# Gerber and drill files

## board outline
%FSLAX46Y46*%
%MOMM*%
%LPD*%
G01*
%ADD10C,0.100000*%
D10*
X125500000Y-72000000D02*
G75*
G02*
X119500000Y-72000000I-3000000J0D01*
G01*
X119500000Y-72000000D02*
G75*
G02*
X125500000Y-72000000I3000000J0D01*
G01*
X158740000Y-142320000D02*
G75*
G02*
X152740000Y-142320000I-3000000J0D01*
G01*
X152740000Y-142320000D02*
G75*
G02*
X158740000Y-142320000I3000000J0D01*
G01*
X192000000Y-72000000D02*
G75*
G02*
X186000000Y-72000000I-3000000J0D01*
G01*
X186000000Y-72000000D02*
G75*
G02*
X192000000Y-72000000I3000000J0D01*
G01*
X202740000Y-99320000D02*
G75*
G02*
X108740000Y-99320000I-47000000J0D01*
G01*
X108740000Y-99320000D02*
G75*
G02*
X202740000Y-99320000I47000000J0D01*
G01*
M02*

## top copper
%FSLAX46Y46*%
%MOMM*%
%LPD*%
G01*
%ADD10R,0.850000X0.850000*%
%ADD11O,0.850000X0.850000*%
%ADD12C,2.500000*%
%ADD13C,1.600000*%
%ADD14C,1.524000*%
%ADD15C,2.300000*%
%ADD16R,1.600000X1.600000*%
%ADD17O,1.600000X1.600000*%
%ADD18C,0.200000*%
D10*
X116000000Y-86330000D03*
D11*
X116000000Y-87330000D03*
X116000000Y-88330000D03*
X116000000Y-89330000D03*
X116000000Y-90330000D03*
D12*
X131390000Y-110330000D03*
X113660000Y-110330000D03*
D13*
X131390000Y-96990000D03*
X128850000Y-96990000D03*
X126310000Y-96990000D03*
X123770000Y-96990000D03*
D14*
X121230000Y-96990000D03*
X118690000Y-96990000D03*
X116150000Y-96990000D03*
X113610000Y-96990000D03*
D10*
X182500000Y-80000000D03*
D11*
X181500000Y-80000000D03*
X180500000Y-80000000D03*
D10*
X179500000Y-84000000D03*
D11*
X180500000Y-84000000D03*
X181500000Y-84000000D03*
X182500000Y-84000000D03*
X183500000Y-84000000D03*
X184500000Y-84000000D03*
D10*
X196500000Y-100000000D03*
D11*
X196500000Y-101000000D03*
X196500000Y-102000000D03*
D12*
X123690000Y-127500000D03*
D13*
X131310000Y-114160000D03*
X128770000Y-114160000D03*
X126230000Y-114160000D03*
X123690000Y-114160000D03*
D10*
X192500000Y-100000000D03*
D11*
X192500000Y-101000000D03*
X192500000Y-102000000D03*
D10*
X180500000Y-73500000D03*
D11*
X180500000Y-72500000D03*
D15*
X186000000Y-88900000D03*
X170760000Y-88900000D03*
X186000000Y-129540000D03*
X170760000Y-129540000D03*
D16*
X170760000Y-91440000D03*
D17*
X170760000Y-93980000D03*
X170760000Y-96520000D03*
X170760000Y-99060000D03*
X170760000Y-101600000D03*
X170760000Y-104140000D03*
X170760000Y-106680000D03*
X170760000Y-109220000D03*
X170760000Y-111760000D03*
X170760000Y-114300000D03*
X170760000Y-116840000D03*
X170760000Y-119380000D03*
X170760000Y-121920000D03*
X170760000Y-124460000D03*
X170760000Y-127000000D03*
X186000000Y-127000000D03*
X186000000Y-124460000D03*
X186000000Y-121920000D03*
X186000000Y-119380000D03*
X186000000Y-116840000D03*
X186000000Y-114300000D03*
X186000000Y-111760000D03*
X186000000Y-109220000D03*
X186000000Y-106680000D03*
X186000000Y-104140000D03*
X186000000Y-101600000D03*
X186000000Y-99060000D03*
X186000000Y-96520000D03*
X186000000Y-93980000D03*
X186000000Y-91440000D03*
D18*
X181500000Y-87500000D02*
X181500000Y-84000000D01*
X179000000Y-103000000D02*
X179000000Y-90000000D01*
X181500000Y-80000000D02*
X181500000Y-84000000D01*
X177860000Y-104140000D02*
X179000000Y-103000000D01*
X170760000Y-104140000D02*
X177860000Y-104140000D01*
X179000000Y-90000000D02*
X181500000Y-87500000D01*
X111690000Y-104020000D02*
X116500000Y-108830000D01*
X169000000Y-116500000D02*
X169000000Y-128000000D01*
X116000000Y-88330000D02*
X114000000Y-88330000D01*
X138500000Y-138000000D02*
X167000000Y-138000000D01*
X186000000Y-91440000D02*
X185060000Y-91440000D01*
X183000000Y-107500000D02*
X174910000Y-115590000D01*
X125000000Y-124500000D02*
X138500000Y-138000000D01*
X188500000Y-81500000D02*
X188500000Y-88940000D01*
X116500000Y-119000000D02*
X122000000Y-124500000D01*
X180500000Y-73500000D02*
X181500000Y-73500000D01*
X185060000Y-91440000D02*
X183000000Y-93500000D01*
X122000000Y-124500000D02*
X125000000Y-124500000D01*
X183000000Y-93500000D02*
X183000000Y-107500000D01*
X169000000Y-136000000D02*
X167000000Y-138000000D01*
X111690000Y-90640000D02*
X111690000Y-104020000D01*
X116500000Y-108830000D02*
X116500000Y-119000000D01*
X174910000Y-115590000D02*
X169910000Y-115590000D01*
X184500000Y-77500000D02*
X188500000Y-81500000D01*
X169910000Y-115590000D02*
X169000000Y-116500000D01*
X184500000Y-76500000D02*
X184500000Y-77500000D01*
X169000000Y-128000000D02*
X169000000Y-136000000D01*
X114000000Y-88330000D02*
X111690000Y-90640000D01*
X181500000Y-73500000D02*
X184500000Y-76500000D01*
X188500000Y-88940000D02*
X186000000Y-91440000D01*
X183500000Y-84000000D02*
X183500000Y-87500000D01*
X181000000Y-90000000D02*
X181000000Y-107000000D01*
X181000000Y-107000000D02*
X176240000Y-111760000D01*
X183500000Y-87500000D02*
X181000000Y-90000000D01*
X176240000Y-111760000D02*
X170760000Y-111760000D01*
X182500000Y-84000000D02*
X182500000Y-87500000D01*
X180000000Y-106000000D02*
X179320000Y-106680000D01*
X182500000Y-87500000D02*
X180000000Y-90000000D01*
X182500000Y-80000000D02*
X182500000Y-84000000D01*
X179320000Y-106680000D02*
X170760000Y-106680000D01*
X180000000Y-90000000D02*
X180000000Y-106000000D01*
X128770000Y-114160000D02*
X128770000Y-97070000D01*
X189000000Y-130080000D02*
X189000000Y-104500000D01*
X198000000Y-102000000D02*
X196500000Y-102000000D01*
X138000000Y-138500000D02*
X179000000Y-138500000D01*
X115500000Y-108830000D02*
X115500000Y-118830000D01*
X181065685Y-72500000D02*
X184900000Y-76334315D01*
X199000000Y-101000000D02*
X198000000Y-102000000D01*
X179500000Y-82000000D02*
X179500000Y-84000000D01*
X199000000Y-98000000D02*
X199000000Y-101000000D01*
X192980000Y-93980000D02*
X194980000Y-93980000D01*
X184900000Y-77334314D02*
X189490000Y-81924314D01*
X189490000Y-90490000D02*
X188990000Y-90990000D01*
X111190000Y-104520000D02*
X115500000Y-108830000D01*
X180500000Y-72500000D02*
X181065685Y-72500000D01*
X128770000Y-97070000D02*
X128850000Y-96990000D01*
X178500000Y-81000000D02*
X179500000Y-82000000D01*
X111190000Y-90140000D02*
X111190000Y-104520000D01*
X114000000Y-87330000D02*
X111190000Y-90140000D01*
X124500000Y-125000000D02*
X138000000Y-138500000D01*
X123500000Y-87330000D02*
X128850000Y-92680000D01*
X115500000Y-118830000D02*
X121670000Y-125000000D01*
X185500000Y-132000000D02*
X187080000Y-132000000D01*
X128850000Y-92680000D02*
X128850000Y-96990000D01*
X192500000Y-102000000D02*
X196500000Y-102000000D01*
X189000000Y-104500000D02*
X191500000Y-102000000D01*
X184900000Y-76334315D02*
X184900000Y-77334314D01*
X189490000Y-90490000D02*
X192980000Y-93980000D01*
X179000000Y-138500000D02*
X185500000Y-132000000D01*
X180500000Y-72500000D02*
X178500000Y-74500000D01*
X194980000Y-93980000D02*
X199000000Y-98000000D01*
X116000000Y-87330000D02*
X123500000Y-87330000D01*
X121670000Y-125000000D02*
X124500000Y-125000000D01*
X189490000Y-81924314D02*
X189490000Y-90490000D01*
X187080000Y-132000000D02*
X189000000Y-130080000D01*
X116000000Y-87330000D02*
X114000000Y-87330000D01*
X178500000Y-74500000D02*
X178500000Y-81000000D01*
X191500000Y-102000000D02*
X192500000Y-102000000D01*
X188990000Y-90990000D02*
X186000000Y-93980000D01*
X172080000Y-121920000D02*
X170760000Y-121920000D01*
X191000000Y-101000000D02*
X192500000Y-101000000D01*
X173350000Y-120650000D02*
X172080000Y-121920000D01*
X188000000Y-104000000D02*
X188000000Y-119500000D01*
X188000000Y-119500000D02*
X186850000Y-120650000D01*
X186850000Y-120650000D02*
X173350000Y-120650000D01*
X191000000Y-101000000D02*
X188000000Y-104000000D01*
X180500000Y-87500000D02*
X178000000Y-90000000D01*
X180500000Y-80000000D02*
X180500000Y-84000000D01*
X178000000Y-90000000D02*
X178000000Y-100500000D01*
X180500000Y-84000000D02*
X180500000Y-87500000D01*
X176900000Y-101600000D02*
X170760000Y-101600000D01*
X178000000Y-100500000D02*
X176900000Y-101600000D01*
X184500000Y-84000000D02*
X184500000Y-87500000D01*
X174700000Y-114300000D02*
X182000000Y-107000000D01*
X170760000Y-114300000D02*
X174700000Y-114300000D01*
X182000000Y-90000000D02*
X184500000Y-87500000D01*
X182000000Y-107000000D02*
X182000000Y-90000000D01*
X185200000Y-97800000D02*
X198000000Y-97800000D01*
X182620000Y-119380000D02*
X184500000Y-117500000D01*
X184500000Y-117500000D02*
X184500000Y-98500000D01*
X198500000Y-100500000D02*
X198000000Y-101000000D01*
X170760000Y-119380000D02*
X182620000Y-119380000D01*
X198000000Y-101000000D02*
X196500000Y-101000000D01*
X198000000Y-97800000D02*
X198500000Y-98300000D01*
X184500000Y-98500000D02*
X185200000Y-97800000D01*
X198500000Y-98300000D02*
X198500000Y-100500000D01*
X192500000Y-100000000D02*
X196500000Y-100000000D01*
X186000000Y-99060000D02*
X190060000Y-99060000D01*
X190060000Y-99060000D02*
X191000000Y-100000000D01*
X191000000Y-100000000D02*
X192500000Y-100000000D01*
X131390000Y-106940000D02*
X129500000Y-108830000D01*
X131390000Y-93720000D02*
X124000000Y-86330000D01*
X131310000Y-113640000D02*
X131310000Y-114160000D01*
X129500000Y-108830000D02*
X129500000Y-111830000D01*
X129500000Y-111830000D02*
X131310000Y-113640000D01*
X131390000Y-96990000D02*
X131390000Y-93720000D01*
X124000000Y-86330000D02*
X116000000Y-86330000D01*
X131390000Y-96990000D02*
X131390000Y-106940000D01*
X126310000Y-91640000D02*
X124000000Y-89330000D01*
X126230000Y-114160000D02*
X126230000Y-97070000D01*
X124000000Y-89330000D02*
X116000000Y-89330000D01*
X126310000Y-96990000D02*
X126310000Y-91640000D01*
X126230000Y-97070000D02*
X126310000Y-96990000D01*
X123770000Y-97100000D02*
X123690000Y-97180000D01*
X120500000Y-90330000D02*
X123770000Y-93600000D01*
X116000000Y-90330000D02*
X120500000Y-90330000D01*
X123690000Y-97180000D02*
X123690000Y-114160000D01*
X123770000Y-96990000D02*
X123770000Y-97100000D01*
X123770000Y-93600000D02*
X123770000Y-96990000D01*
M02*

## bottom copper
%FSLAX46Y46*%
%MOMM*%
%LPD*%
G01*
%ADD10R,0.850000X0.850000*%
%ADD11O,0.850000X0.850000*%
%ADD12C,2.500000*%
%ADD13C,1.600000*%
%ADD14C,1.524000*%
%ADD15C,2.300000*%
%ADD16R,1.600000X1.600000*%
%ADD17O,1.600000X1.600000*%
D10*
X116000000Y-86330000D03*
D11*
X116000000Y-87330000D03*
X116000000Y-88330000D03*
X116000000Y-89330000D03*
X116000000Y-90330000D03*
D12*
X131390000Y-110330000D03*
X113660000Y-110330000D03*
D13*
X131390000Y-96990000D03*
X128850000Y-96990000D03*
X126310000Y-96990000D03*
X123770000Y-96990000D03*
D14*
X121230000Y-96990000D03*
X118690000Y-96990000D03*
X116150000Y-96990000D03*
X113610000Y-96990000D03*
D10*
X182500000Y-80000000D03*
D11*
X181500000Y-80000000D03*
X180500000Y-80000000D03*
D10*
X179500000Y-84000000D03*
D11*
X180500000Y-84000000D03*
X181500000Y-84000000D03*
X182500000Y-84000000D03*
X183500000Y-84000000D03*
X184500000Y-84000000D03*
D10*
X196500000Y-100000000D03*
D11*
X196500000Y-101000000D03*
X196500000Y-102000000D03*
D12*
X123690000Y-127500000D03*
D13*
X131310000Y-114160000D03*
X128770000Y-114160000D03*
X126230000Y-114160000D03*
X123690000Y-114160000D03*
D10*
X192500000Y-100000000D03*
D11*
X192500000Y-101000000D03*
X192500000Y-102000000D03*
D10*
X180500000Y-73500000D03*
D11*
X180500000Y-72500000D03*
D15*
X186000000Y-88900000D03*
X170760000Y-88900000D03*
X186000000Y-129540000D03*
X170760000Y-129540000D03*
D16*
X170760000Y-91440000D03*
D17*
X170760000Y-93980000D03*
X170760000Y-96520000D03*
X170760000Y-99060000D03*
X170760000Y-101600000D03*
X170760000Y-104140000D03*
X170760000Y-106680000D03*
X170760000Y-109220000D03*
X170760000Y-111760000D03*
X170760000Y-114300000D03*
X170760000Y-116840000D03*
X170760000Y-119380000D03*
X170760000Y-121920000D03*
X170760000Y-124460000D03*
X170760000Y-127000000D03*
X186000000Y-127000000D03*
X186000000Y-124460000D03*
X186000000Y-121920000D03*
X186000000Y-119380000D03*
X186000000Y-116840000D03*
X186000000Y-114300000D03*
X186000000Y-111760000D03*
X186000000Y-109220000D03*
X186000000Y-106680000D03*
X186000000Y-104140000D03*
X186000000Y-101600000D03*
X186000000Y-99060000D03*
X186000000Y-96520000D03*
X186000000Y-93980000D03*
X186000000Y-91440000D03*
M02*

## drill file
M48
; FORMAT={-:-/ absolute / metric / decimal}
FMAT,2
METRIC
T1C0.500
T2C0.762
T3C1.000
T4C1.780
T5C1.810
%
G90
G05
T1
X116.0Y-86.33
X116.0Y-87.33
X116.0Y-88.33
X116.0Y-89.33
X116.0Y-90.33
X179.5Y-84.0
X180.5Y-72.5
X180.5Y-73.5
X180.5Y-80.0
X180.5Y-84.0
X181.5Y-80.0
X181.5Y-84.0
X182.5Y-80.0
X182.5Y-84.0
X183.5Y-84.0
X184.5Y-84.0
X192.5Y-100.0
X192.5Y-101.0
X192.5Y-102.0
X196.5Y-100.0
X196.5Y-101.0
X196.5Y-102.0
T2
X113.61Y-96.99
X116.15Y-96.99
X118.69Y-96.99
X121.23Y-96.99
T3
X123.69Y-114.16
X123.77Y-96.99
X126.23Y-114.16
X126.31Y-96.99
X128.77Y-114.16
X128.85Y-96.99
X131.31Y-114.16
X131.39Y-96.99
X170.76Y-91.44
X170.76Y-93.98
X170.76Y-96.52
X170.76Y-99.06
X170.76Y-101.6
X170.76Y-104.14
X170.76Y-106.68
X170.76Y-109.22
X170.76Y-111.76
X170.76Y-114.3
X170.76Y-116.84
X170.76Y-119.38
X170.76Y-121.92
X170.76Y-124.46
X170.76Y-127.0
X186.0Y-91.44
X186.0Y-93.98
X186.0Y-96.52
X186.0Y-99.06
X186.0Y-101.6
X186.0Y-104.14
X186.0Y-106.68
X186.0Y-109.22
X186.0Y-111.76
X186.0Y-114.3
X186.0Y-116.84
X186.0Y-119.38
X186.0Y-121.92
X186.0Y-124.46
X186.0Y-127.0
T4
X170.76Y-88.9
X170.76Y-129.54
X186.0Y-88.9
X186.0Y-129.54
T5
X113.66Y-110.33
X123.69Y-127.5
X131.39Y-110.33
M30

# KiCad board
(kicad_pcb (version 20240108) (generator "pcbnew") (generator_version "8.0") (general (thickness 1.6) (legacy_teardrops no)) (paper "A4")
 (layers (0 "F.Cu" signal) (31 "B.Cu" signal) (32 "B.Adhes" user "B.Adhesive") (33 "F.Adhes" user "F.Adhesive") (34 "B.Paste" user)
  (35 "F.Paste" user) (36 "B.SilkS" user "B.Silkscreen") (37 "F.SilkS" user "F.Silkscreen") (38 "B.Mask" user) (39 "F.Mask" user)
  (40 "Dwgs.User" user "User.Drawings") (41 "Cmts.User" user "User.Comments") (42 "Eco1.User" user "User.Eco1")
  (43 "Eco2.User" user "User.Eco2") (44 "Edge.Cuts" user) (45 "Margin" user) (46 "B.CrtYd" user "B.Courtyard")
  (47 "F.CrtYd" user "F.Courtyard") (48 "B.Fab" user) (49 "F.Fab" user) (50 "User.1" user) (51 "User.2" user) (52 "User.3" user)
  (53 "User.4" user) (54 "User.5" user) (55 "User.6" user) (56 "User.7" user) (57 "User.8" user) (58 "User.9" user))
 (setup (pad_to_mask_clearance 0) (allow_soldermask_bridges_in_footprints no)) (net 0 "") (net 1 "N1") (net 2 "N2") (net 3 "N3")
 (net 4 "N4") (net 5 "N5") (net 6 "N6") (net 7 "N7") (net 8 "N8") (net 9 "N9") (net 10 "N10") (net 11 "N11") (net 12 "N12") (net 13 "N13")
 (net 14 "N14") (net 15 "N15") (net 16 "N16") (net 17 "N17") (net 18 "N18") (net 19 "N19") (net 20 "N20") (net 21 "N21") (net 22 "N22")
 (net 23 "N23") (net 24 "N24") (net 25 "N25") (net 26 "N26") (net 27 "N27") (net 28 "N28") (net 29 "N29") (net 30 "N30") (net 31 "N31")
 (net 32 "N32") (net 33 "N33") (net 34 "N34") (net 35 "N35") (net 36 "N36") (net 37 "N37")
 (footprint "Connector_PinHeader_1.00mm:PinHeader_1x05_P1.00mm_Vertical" (layer "F.Cu") (at 116 86.33)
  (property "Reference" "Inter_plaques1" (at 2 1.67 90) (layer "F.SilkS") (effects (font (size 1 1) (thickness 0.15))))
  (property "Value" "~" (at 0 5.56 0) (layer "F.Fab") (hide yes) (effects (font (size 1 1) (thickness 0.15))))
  (pad "1" thru_hole rect (at 0 0) (size 0.85 0.85) (drill 0.5) (layers "*.Cu" "*.Mask") (remove_unused_layers no) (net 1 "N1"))
  (pad "2" thru_hole oval (at 0 1) (size 0.85 0.85) (drill 0.5) (layers "*.Cu" "*.Mask") (remove_unused_layers no) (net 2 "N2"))
  (pad "3" thru_hole oval (at 0 2) (size 0.85 0.85) (drill 0.5) (layers "*.Cu" "*.Mask") (remove_unused_layers no) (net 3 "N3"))
  (pad "4" thru_hole oval (at 0 3) (size 0.85 0.85) (drill 0.5) (layers "*.Cu" "*.Mask") (remove_unused_layers no) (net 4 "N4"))
  (pad "5" thru_hole oval (at 0 4) (size 0.85 0.85) (drill 0.5) (layers "*.Cu" "*.Mask") (remove_unused_layers no) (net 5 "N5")))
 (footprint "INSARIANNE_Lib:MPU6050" (layer "F.Cu") (at 131.39 96.99 180)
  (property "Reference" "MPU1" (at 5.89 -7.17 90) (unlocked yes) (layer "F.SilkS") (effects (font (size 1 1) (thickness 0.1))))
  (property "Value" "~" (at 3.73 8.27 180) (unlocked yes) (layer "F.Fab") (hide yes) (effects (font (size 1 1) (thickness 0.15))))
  (pad "" np_thru_hole circle (at 0 -13.34 180) (size 2.5 2.5) (drill 1.81) (layers "F&B.Cu" "*.Mask"))
  (pad "" np_thru_hole circle (at 17.73 -13.34 180) (size 2.5 2.5) (drill 1.81) (layers "F&B.Cu" "*.Mask"))
  (pad "1" thru_hole circle (at 0 0 180) (size 1.6 1.6) (drill 1) (layers "*.Cu" "*.Mask") (remove_unused_layers no) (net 1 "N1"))
  (pad "2" thru_hole circle (at 2.54 0 180) (size 1.6 1.6) (drill 1) (layers "*.Cu" "*.Mask") (remove_unused_layers no) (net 2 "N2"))
  (pad "3" thru_hole circle (at 5.08 0 180) (size 1.6 1.6) (drill 1) (layers "*.Cu" "*.Mask") (remove_unused_layers no) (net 4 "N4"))
  (pad "4" thru_hole circle (at 7.62 0 180) (size 1.6 1.6) (drill 1) (layers "*.Cu" "*.Mask") (remove_unused_layers no) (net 5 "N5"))
  (pad "5" thru_hole circle (at 10.16 0 180) (size 1.524 1.524) (drill 0.762) (layers "*.Cu" "*.Mask") (remove_unused_layers no)
   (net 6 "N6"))
  (pad "6" thru_hole circle (at 12.7 0 180) (size 1.524 1.524) (drill 0.762) (layers "*.Cu" "*.Mask") (remove_unused_layers no) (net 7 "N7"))
  (pad "7" thru_hole circle (at 15.24 0 180) (size 1.524 1.524) (drill 0.762) (layers "*.Cu" "*.Mask") (remove_unused_layers no)
   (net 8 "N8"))
  (pad "8" thru_hole circle (at 17.78 0 180) (size 1.524 1.524) (drill 0.762) (layers "*.Cu" "*.Mask") (remove_unused_layers no)
   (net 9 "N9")))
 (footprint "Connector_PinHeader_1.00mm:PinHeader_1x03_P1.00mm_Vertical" (layer "F.Cu") (at 182.5 80 -90)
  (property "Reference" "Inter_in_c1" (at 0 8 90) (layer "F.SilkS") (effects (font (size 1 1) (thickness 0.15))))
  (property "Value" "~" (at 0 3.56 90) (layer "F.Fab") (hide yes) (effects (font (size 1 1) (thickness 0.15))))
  (pad "1" thru_hole rect (at 0 0 270) (size 0.85 0.85) (drill 0.5) (layers "*.Cu" "*.Mask") (remove_unused_layers no) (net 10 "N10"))
  (pad "2" thru_hole oval (at 0 1 270) (size 0.85 0.85) (drill 0.5) (layers "*.Cu" "*.Mask") (remove_unused_layers no) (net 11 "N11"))
  (pad "3" thru_hole oval (at 0 2 270) (size 0.85 0.85) (drill 0.5) (layers "*.Cu" "*.Mask") (remove_unused_layers no) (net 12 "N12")))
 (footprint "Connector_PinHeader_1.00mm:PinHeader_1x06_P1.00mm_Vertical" (layer "F.Cu") (at 179.5 84 90)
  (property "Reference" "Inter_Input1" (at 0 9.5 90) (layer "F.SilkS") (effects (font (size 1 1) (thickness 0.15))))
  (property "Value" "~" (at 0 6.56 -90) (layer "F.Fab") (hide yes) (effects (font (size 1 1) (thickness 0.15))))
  (pad "1" thru_hole rect (at 0 0 90) (size 0.85 0.85) (drill 0.5) (layers "*.Cu" "*.Mask") (remove_unused_layers no) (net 2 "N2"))
  (pad "2" thru_hole oval (at 0 1 90) (size 0.85 0.85) (drill 0.5) (layers "*.Cu" "*.Mask") (remove_unused_layers no) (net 12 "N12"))
  (pad "3" thru_hole oval (at 0 2 90) (size 0.85 0.85) (drill 0.5) (layers "*.Cu" "*.Mask") (remove_unused_layers no) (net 11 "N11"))
  (pad "4" thru_hole oval (at 0 3 90) (size 0.85 0.85) (drill 0.5) (layers "*.Cu" "*.Mask") (remove_unused_layers no) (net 10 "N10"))
  (pad "5" thru_hole oval (at 0 4 90) (size 0.85 0.85) (drill 0.5) (layers "*.Cu" "*.Mask") (remove_unused_layers no) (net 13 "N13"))
  (pad "6" thru_hole oval (at 0 5 90) (size 0.85 0.85) (drill 0.5) (layers "*.Cu" "*.Mask") (remove_unused_layers no) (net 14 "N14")))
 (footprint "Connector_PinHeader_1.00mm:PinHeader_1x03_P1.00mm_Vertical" (layer "F.Cu") (at 196.5 100)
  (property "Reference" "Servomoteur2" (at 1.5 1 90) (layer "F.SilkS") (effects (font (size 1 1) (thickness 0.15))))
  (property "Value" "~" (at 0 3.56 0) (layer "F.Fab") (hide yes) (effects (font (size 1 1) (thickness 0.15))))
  (pad "1" thru_hole rect (at 0 0) (size 0.85 0.85) (drill 0.5) (layers "*.Cu" "*.Mask") (remove_unused_layers no) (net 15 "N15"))
  (pad "2" thru_hole oval (at 0 1) (size 0.85 0.85) (drill 0.5) (layers "*.Cu" "*.Mask") (remove_unused_layers no) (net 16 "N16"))
  (pad "3" thru_hole oval (at 0 2) (size 0.85 0.85) (drill 0.5) (layers "*.Cu" "*.Mask") (remove_unused_layers no) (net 2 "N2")))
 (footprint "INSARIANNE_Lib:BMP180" (layer "F.Cu") (at 131.31 114.16 180)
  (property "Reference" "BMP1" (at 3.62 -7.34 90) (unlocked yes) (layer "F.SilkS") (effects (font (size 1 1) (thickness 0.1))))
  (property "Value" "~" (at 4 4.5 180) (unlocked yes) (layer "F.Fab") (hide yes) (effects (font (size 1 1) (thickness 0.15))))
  (pad "" np_thru_hole circle (at 7.62 -13.34 180) (size 2.5 2.5) (drill 1.81) (layers "F&B.Cu" "*.Mask"))
  (pad "1" thru_hole circle (at 0 0 180) (size 1.6 1.6) (drill 1) (layers "*.Cu" "*.Mask") (remove_unused_layers no) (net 1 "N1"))
  (pad "2" thru_hole circle (at 2.54 0 180) (size 1.6 1.6) (drill 1) (layers "*.Cu" "*.Mask") (remove_unused_layers no) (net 2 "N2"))
  (pad "3" thru_hole circle (at 5.08 0 180) (size 1.6 1.6) (drill 1) (layers "*.Cu" "*.Mask") (remove_unused_layers no) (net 4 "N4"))
  (pad "4" thru_hole circle (at 7.62 0 180) (size 1.6 1.6) (drill 1) (layers "*.Cu" "*.Mask") (remove_unused_layers no) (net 5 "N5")))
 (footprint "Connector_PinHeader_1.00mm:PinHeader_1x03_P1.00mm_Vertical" (layer "F.Cu") (at 192.5 100)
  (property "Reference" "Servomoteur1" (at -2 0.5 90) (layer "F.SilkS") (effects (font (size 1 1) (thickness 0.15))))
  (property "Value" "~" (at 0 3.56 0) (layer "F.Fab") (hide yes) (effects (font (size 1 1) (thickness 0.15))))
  (pad "1" thru_hole rect (at 0 0) (size 0.85 0.85) (drill 0.5) (layers "*.Cu" "*.Mask") (remove_unused_layers no) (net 15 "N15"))
  (pad "2" thru_hole oval (at 0 1) (size 0.85 0.85) (drill 0.5) (layers "*.Cu" "*.Mask") (remove_unused_layers no) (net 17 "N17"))
  (pad "3" thru_hole oval (at 0 2) (size 0.85 0.85) (drill 0.5) (layers "*.Cu" "*.Mask") (remove_unused_layers no) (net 2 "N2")))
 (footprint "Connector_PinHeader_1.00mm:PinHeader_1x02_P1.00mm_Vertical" (layer "F.Cu") (at 180.5 73.5 180)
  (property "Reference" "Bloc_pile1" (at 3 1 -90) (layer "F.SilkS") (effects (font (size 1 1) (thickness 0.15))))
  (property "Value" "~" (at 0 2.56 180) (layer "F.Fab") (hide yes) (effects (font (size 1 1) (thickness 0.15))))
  (pad "1" thru_hole rect (at 0 0 180) (size 0.85 0.85) (drill 0.5) (layers "*.Cu" "*.Mask") (remove_unused_layers no) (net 3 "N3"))
  (pad "2" thru_hole oval (at 0 1 180) (size 0.85 0.85) (drill 0.5) (layers "*.Cu" "*.Mask") (remove_unused_layers no) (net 2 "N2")))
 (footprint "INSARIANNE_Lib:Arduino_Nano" (layer "F.Cu") (at 170.76 91.44 -90)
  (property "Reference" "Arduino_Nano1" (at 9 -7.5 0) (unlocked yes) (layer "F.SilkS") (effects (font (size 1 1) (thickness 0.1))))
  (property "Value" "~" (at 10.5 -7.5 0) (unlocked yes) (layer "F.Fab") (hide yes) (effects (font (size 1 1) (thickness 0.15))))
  (pad "" np_thru_hole circle (at -2.54 -15.24 270) (size 2.3 2.3) (drill 1.78) (layers "F&B.Cu" "*.Mask"))
  (pad "" np_thru_hole circle (at -2.54 0 270) (size 2.3 2.3) (drill 1.78) (layers "F&B.Cu" "*.Mask"))
  (pad "" np_thru_hole circle (at 38.1 -15.24 270) (size 2.3 2.3) (drill 1.78) (layers "F&B.Cu" "*.Mask"))
  (pad "" np_thru_hole circle (at 38.1 0 270) (size 2.3 2.3) (drill 1.78) (layers "F&B.Cu" "*.Mask"))
  (pad "1" thru_hole rect (at 0 0) (size 1.6 1.6) (drill 1) (layers "*.Cu" "*.Mask") (remove_unused_layers no) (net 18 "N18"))
  (pad "2" thru_hole oval (at 2.54 0) (size 1.6 1.6) (drill 1) (layers "*.Cu" "*.Mask") (remove_unused_layers no) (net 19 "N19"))
  (pad "3" thru_hole oval (at 5.08 0) (size 1.6 1.6) (drill 1) (layers "*.Cu" "*.Mask") (remove_unused_layers no) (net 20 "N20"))
  (pad "4" thru_hole oval (at 7.62 0) (size 1.6 1.6) (drill 1) (layers "*.Cu" "*.Mask") (remove_unused_layers no) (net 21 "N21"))
  (pad "5" thru_hole oval (at 10.16 0) (size 1.6 1.6) (drill 1) (layers "*.Cu" "*.Mask") (remove_unused_layers no) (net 12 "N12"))
  (pad "6" thru_hole oval (at 12.7 0) (size 1.6 1.6) (drill 1) (layers "*.Cu" "*.Mask") (remove_unused_layers no) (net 11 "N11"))
  (pad "7" thru_hole oval (at 15.24 0) (size 1.6 1.6) (drill 1) (layers "*.Cu" "*.Mask") (remove_unused_layers no) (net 10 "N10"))
  (pad "8" thru_hole oval (at 17.78 0) (size 1.6 1.6) (drill 1) (layers "*.Cu" "*.Mask") (remove_unused_layers no) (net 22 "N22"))
  (pad "9" thru_hole oval (at 20.32 0) (size 1.6 1.6) (drill 1) (layers "*.Cu" "*.Mask") (remove_unused_layers no) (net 13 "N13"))
  (pad "10" thru_hole oval (at 22.86 0) (size 1.6 1.6) (drill 1) (layers "*.Cu" "*.Mask") (remove_unused_layers no) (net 14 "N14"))
  (pad "11" thru_hole oval (at 25.4 0) (size 1.6 1.6) (drill 1) (layers "*.Cu" "*.Mask") (remove_unused_layers no) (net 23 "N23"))
  (pad "12" thru_hole oval (at 27.94 0) (size 1.6 1.6) (drill 1) (layers "*.Cu" "*.Mask") (remove_unused_layers no) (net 16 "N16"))
  (pad "13" thru_hole oval (at 30.48 0) (size 1.6 1.6) (drill 1) (layers "*.Cu" "*.Mask") (remove_unused_layers no) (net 17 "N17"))
  (pad "14" thru_hole oval (at 33.02 0) (size 1.6 1.6) (drill 1) (layers "*.Cu" "*.Mask") (remove_unused_layers no) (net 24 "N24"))
  (pad "15" thru_hole oval (at 35.56 0) (size 1.6 1.6) (drill 1) (layers "*.Cu" "*.Mask") (remove_unused_layers no) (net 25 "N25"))
  (pad "16" thru_hole oval (at 35.56 -15.24) (size 1.6 1.6) (drill 1) (layers "*.Cu" "*.Mask") (remove_unused_layers no) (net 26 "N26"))
  (pad "17" thru_hole oval (at 33.02 -15.24) (size 1.6 1.6) (drill 1) (layers "*.Cu" "*.Mask") (remove_unused_layers no) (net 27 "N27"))
  (pad "18" thru_hole oval (at 30.48 -15.24) (size 1.6 1.6) (drill 1) (layers "*.Cu" "*.Mask") (remove_unused_layers no) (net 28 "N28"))
  (pad "19" thru_hole oval (at 27.94 -15.24) (size 1.6 1.6) (drill 1) (layers "*.Cu" "*.Mask") (remove_unused_layers no) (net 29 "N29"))
  (pad "20" thru_hole oval (at 25.4 -15.24) (size 1.6 1.6) (drill 1) (layers "*.Cu" "*.Mask") (remove_unused_layers no) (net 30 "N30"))
  (pad "21" thru_hole oval (at 22.86 -15.24) (size 1.6 1.6) (drill 1) (layers "*.Cu" "*.Mask") (remove_unused_layers no) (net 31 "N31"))
  (pad "22" thru_hole oval (at 20.32 -15.24) (size 1.6 1.6) (drill 1) (layers "*.Cu" "*.Mask") (remove_unused_layers no) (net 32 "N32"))
  (pad "23" thru_hole oval (at 17.78 -15.24) (size 1.6 1.6) (drill 1) (layers "*.Cu" "*.Mask") (remove_unused_layers no) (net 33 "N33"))
  (pad "24" thru_hole oval (at 15.24 -15.24) (size 1.6 1.6) (drill 1) (layers "*.Cu" "*.Mask") (remove_unused_layers no) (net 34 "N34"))
  (pad "25" thru_hole oval (at 12.7 -15.24) (size 1.6 1.6) (drill 1) (layers "*.Cu" "*.Mask") (remove_unused_layers no) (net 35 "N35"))
  (pad "26" thru_hole oval (at 10.16 -15.24) (size 1.6 1.6) (drill 1) (layers "*.Cu" "*.Mask") (remove_unused_layers no) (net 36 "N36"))
  (pad "27" thru_hole oval (at 7.62 -15.24) (size 1.6 1.6) (drill 1) (layers "*.Cu" "*.Mask") (remove_unused_layers no) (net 15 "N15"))
  (pad "28" thru_hole oval (at 5.08 -15.24) (size 1.6 1.6) (drill 1) (layers "*.Cu" "*.Mask") (remove_unused_layers no) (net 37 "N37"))
  (pad "29" thru_hole oval (at 2.54 -15.24) (size 1.6 1.6) (drill 1) (layers "*.Cu" "*.Mask") (remove_unused_layers no) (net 2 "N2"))
  (pad "30" thru_hole oval (at 0 -15.24) (size 1.6 1.6) (drill 1) (layers "*.Cu" "*.Mask") (remove_unused_layers no) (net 3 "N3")))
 (gr_circle (center 122.5 72) (end 125.5 72) (stroke (width 0.1) (type default)) (fill none) (layer "Edge.Cuts"))
 (gr_circle (center 155.74 142.32) (end 158.74 142.32) (stroke (width 0.1) (type default)) (fill none) (layer "Edge.Cuts"))
 (gr_circle (center 189 72) (end 192 72) (stroke (width 0.1) (type default)) (fill none) (layer "Edge.Cuts"))
 (gr_circle (center 155.74 99.32) (end 202.74 99.32) (stroke (width 0.1) (type default)) (fill none) (layer "Edge.Cuts"))
 (segment (start 181.5 87.5) (end 181.5 84) (width 0.2) (layer "F.Cu") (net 11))
 (segment (start 179 103) (end 179 90) (width 0.2) (layer "F.Cu") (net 11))
 (segment (start 181.5 80) (end 181.5 84) (width 0.2) (layer "F.Cu") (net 11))
 (segment (start 177.86 104.14) (end 179 103) (width 0.2) (layer "F.Cu") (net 11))
 (segment (start 170.76 104.14) (end 177.86 104.14) (width 0.2) (layer "F.Cu") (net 11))
 (segment (start 179 90) (end 181.5 87.5) (width 0.2) (layer "F.Cu") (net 11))
 (segment (start 111.69 104.02) (end 116.5 108.83) (width 0.2) (layer "F.Cu") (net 3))
 (segment (start 169 116.5) (end 169 128) (width 0.2) (layer "F.Cu") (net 3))
 (segment (start 116 88.33) (end 114 88.33) (width 0.2) (layer "F.Cu") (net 3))
 (segment (start 138.5 138) (end 167 138) (width 0.2) (layer "F.Cu") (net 3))
 (segment (start 186 91.44) (end 185.06 91.44) (width 0.2) (layer "F.Cu") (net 3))
 (segment (start 183 107.5) (end 174.91 115.59) (width 0.2) (layer "F.Cu") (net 3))
 (segment (start 125 124.5) (end 138.5 138) (width 0.2) (layer "F.Cu") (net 3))
 (segment (start 188.5 81.5) (end 188.5 88.94) (width 0.2) (layer "F.Cu") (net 3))
 (segment (start 116.5 119) (end 122 124.5) (width 0.2) (layer "F.Cu") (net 3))
 (segment (start 180.5 73.5) (end 181.5 73.5) (width 0.2) (layer "F.Cu") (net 3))
 (segment (start 185.06 91.44) (end 183 93.5) (width 0.2) (layer "F.Cu") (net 3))
 (segment (start 122 124.5) (end 125 124.5) (width 0.2) (layer "F.Cu") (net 3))
 (segment (start 183 93.5) (end 183 107.5) (width 0.2) (layer "F.Cu") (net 3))
 (segment (start 169 136) (end 167 138) (width 0.2) (layer "F.Cu") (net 3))
 (segment (start 111.69 90.64) (end 111.69 104.02) (width 0.2) (layer "F.Cu") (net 3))
 (segment (start 116.5 108.83) (end 116.5 119) (width 0.2) (layer "F.Cu") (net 3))
 (segment (start 174.91 115.59) (end 169.91 115.59) (width 0.2) (layer "F.Cu") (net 3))
 (segment (start 184.5 77.5) (end 188.5 81.5) (width 0.2) (layer "F.Cu") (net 3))
 (segment (start 169.91 115.59) (end 169 116.5) (width 0.2) (layer "F.Cu") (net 3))
 (segment (start 184.5 76.5) (end 184.5 77.5) (width 0.2) (layer "F.Cu") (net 3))
 (segment (start 169 128) (end 169 136) (width 0.2) (layer "F.Cu") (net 3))
 (segment (start 114 88.33) (end 111.69 90.64) (width 0.2) (layer "F.Cu") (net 3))
 (segment (start 181.5 73.5) (end 184.5 76.5) (width 0.2) (layer "F.Cu") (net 3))
 (segment (start 188.5 88.94) (end 186 91.44) (width 0.2) (layer "F.Cu") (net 3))
 (segment (start 183.5 84) (end 183.5 87.5) (width 0.2) (layer "F.Cu") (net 13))
 (segment (start 181 90) (end 181 107) (width 0.2) (layer "F.Cu") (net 13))
 (segment (start 181 107) (end 176.24 111.76) (width 0.2) (layer "F.Cu") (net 13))
 (segment (start 183.5 87.5) (end 181 90) (width 0.2) (layer "F.Cu") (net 13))
 (segment (start 176.24 111.76) (end 170.76 111.76) (width 0.2) (layer "F.Cu") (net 13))
 (segment (start 182.5 84) (end 182.5 87.5) (width 0.2) (layer "F.Cu") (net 10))
 (segment (start 180 106) (end 179.32 106.68) (width 0.2) (layer "F.Cu") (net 10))
 (segment (start 182.5 87.5) (end 180 90) (width 0.2) (layer "F.Cu") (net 10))
 (segment (start 182.5 80) (end 182.5 84) (width 0.2) (layer "F.Cu") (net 10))
 (segment (start 179.32 106.68) (end 170.76 106.68) (width 0.2) (layer "F.Cu") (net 10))
 (segment (start 180 90) (end 180 106) (width 0.2) (layer "F.Cu") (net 10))
 (segment (start 128.77 114.16) (end 128.77 97.07) (width 0.2) (layer "F.Cu") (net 2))
 (segment (start 189 130.08) (end 189 104.5) (width 0.2) (layer "F.Cu") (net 2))
 (segment (start 198 102) (end 196.5 102) (width 0.2) (layer "F.Cu") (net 2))
 (segment (start 138 138.5) (end 179 138.5) (width 0.2) (layer "F.Cu") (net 2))
 (segment (start 115.5 108.83) (end 115.5 118.83) (width 0.2) (layer "F.Cu") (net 2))
 (segment (start 181.065685 72.5) (end 184.9 76.334315) (width 0.2) (layer "F.Cu") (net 2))
 (segment (start 199 101) (end 198 102) (width 0.2) (layer "F.Cu") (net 2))
 (segment (start 179.5 82) (end 179.5 84) (width 0.2) (layer "F.Cu") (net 2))
 (segment (start 199 98) (end 199 101) (width 0.2) (layer "F.Cu") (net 2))
 (segment (start 192.98 93.98) (end 194.98 93.98) (width 0.2) (layer "F.Cu") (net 2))
 (segment (start 184.9 77.334314) (end 189.49 81.924314) (width 0.2) (layer "F.Cu") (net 2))
 (segment (start 189.49 90.49) (end 188.99 90.99) (width 0.2) (layer "F.Cu") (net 2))
 (segment (start 111.19 104.52) (end 115.5 108.83) (width 0.2) (layer "F.Cu") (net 2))
 (segment (start 180.5 72.5) (end 181.065685 72.5) (width 0.2) (layer "F.Cu") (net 2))
 (segment (start 128.77 97.07) (end 128.85 96.99) (width 0.2) (layer "F.Cu") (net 2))
 (segment (start 178.5 81) (end 179.5 82) (width 0.2) (layer "F.Cu") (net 2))
 (segment (start 111.19 90.14) (end 111.19 104.52) (width 0.2) (layer "F.Cu") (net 2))
 (segment (start 114 87.33) (end 111.19 90.14) (width 0.2) (layer "F.Cu") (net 2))
 (segment (start 124.5 125) (end 138 138.5) (width 0.2) (layer "F.Cu") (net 2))
 (segment (start 123.5 87.33) (end 128.85 92.68) (width 0.2) (layer "F.Cu") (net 2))
 (segment (start 115.5 118.83) (end 121.67 125) (width 0.2) (layer "F.Cu") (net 2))
 (segment (start 185.5 132) (end 187.08 132) (width 0.2) (layer "F.Cu") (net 2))
 (segment (start 128.85 92.68) (end 128.85 96.99) (width 0.2) (layer "F.Cu") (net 2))
 (segment (start 192.5 102) (end 196.5 102) (width 0.2) (layer "F.Cu") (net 2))
 (segment (start 189 104.5) (end 191.5 102) (width 0.2) (layer "F.Cu") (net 2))
 (segment (start 184.9 76.334315) (end 184.9 77.334314) (width 0.2) (layer "F.Cu") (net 2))
 (segment (start 189.49 90.49) (end 192.98 93.98) (width 0.2) (layer "F.Cu") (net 2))
 (segment (start 179 138.5) (end 185.5 132) (width 0.2) (layer "F.Cu") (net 2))
 (segment (start 180.5 72.5) (end 178.5 74.5) (width 0.2) (layer "F.Cu") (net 2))
 (segment (start 194.98 93.98) (end 199 98) (width 0.2) (layer "F.Cu") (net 2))
 (segment (start 116 87.33) (end 123.5 87.33) (width 0.2) (layer "F.Cu") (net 2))
 (segment (start 121.67 125) (end 124.5 125) (width 0.2) (layer "F.Cu") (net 2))
 (segment (start 189.49 81.924314) (end 189.49 90.49) (width 0.2) (layer "F.Cu") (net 2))
 (segment (start 187.08 132) (end 189 130.08) (width 0.2) (layer "F.Cu") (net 2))
 (segment (start 116 87.33) (end 114 87.33) (width 0.2) (layer "F.Cu") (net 2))
 (segment (start 178.5 74.5) (end 178.5 81) (width 0.2) (layer "F.Cu") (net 2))
 (segment (start 191.5 102) (end 192.5 102) (width 0.2) (layer "F.Cu") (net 2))
 (segment (start 188.99 90.99) (end 186 93.98) (width 0.2) (layer "F.Cu") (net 2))
 (segment (start 172.08 121.92) (end 170.76 121.92) (width 0.2) (layer "F.Cu") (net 17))
 (segment (start 191 101) (end 192.5 101) (width 0.2) (layer "F.Cu") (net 17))
 (segment (start 173.35 120.65) (end 172.08 121.92) (width 0.2) (layer "F.Cu") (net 17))
 (segment (start 188 104) (end 188 119.5) (width 0.2) (layer "F.Cu") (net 17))
 (segment (start 188 119.5) (end 186.85 120.65) (width 0.2) (layer "F.Cu") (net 17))
 (segment (start 186.85 120.65) (end 173.35 120.65) (width 0.2) (layer "F.Cu") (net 17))
 (segment (start 191 101) (end 188 104) (width 0.2) (layer "F.Cu") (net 17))
 (segment (start 180.5 87.5) (end 178 90) (width 0.2) (layer "F.Cu") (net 12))
 (segment (start 180.5 80) (end 180.5 84) (width 0.2) (layer "F.Cu") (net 12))
 (segment (start 178 90) (end 178 100.5) (width 0.2) (layer "F.Cu") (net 12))
 (segment (start 180.5 84) (end 180.5 87.5) (width 0.2) (layer "F.Cu") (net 12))
 (segment (start 176.9 101.6) (end 170.76 101.6) (width 0.2) (layer "F.Cu") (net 12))
 (segment (start 178 100.5) (end 176.9 101.6) (width 0.2) (layer "F.Cu") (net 12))
 (segment (start 184.5 84) (end 184.5 87.5) (width 0.2) (layer "F.Cu") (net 14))
 (segment (start 174.7 114.3) (end 182 107) (width 0.2) (layer "F.Cu") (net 14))
 (segment (start 170.76 114.3) (end 174.7 114.3) (width 0.2) (layer "F.Cu") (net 14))
 (segment (start 182 90) (end 184.5 87.5) (width 0.2) (layer "F.Cu") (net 14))
 (segment (start 182 107) (end 182 90) (width 0.2) (layer "F.Cu") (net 14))
 (segment (start 185.2 97.8) (end 198 97.8) (width 0.2) (layer "F.Cu") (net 16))
 (segment (start 182.62 119.38) (end 184.5 117.5) (width 0.2) (layer "F.Cu") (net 16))
 (segment (start 184.5 117.5) (end 184.5 98.5) (width 0.2) (layer "F.Cu") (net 16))
 (segment (start 198.5 100.5) (end 198 101) (width 0.2) (layer "F.Cu") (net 16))
 (segment (start 170.76 119.38) (end 182.62 119.38) (width 0.2) (layer "F.Cu") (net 16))
 (segment (start 198 101) (end 196.5 101) (width 0.2) (layer "F.Cu") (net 16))
 (segment (start 198 97.8) (end 198.5 98.3) (width 0.2) (layer "F.Cu") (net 16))
 (segment (start 184.5 98.5) (end 185.2 97.8) (width 0.2) (layer "F.Cu") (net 16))
 (segment (start 198.5 98.3) (end 198.5 100.5) (width 0.2) (layer "F.Cu") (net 16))
 (segment (start 192.5 100) (end 196.5 100) (width 0.2) (layer "F.Cu") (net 15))
 (segment (start 186 99.06) (end 190.06 99.06) (width 0.2) (layer "F.Cu") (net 15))
 (segment (start 190.06 99.06) (end 191 100) (width 0.2) (layer "F.Cu") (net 15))
 (segment (start 191 100) (end 192.5 100) (width 0.2) (layer "F.Cu") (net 15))
 (segment (start 131.39 106.94) (end 129.5 108.83) (width 0.2) (layer "F.Cu") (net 1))
 (segment (start 131.39 93.72) (end 124 86.33) (width 0.2) (layer "F.Cu") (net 1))
 (segment (start 131.31 113.64) (end 131.31 114.16) (width 0.2) (layer "F.Cu") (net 1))
 (segment (start 129.5 108.83) (end 129.5 111.83) (width 0.2) (layer "F.Cu") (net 1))
 (segment (start 129.5 111.83) (end 131.31 113.64) (width 0.2) (layer "F.Cu") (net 1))
 (segment (start 131.39 96.99) (end 131.39 93.72) (width 0.2) (layer "F.Cu") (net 1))
 (segment (start 124 86.33) (end 116 86.33) (width 0.2) (layer "F.Cu") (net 1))
 (segment (start 131.39 96.99) (end 131.39 106.94) (width 0.2) (layer "F.Cu") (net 1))
 (segment (start 126.31 91.64) (end 124 89.33) (width 0.2) (layer "F.Cu") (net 4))
 (segment (start 126.23 114.16) (end 126.23 97.07) (width 0.2) (layer "F.Cu") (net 4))
 (segment (start 124 89.33) (end 116 89.33) (width 0.2) (layer "F.Cu") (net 4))
 (segment (start 126.31 96.99) (end 126.31 91.64) (width 0.2) (layer "F.Cu") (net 4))
 (segment (start 126.23 97.07) (end 126.31 96.99) (width 0.2) (layer "F.Cu") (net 4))
 (segment (start 123.77 97.1) (end 123.69 97.18) (width 0.2) (layer "F.Cu") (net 5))
 (segment (start 120.5 90.33) (end 123.77 93.6) (width 0.2) (layer "F.Cu") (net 5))
 (segment (start 116 90.33) (end 120.5 90.33) (width 0.2) (layer "F.Cu") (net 5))
 (segment (start 123.69 97.18) (end 123.69 114.16) (width 0.2) (layer "F.Cu") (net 5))
 (segment (start 123.77 96.99) (end 123.77 97.1) (width 0.2) (layer "F.Cu") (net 5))
 (segment (start 123.77 93.6) (end 123.77 96.99) (width 0.2) (layer "F.Cu") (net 5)))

